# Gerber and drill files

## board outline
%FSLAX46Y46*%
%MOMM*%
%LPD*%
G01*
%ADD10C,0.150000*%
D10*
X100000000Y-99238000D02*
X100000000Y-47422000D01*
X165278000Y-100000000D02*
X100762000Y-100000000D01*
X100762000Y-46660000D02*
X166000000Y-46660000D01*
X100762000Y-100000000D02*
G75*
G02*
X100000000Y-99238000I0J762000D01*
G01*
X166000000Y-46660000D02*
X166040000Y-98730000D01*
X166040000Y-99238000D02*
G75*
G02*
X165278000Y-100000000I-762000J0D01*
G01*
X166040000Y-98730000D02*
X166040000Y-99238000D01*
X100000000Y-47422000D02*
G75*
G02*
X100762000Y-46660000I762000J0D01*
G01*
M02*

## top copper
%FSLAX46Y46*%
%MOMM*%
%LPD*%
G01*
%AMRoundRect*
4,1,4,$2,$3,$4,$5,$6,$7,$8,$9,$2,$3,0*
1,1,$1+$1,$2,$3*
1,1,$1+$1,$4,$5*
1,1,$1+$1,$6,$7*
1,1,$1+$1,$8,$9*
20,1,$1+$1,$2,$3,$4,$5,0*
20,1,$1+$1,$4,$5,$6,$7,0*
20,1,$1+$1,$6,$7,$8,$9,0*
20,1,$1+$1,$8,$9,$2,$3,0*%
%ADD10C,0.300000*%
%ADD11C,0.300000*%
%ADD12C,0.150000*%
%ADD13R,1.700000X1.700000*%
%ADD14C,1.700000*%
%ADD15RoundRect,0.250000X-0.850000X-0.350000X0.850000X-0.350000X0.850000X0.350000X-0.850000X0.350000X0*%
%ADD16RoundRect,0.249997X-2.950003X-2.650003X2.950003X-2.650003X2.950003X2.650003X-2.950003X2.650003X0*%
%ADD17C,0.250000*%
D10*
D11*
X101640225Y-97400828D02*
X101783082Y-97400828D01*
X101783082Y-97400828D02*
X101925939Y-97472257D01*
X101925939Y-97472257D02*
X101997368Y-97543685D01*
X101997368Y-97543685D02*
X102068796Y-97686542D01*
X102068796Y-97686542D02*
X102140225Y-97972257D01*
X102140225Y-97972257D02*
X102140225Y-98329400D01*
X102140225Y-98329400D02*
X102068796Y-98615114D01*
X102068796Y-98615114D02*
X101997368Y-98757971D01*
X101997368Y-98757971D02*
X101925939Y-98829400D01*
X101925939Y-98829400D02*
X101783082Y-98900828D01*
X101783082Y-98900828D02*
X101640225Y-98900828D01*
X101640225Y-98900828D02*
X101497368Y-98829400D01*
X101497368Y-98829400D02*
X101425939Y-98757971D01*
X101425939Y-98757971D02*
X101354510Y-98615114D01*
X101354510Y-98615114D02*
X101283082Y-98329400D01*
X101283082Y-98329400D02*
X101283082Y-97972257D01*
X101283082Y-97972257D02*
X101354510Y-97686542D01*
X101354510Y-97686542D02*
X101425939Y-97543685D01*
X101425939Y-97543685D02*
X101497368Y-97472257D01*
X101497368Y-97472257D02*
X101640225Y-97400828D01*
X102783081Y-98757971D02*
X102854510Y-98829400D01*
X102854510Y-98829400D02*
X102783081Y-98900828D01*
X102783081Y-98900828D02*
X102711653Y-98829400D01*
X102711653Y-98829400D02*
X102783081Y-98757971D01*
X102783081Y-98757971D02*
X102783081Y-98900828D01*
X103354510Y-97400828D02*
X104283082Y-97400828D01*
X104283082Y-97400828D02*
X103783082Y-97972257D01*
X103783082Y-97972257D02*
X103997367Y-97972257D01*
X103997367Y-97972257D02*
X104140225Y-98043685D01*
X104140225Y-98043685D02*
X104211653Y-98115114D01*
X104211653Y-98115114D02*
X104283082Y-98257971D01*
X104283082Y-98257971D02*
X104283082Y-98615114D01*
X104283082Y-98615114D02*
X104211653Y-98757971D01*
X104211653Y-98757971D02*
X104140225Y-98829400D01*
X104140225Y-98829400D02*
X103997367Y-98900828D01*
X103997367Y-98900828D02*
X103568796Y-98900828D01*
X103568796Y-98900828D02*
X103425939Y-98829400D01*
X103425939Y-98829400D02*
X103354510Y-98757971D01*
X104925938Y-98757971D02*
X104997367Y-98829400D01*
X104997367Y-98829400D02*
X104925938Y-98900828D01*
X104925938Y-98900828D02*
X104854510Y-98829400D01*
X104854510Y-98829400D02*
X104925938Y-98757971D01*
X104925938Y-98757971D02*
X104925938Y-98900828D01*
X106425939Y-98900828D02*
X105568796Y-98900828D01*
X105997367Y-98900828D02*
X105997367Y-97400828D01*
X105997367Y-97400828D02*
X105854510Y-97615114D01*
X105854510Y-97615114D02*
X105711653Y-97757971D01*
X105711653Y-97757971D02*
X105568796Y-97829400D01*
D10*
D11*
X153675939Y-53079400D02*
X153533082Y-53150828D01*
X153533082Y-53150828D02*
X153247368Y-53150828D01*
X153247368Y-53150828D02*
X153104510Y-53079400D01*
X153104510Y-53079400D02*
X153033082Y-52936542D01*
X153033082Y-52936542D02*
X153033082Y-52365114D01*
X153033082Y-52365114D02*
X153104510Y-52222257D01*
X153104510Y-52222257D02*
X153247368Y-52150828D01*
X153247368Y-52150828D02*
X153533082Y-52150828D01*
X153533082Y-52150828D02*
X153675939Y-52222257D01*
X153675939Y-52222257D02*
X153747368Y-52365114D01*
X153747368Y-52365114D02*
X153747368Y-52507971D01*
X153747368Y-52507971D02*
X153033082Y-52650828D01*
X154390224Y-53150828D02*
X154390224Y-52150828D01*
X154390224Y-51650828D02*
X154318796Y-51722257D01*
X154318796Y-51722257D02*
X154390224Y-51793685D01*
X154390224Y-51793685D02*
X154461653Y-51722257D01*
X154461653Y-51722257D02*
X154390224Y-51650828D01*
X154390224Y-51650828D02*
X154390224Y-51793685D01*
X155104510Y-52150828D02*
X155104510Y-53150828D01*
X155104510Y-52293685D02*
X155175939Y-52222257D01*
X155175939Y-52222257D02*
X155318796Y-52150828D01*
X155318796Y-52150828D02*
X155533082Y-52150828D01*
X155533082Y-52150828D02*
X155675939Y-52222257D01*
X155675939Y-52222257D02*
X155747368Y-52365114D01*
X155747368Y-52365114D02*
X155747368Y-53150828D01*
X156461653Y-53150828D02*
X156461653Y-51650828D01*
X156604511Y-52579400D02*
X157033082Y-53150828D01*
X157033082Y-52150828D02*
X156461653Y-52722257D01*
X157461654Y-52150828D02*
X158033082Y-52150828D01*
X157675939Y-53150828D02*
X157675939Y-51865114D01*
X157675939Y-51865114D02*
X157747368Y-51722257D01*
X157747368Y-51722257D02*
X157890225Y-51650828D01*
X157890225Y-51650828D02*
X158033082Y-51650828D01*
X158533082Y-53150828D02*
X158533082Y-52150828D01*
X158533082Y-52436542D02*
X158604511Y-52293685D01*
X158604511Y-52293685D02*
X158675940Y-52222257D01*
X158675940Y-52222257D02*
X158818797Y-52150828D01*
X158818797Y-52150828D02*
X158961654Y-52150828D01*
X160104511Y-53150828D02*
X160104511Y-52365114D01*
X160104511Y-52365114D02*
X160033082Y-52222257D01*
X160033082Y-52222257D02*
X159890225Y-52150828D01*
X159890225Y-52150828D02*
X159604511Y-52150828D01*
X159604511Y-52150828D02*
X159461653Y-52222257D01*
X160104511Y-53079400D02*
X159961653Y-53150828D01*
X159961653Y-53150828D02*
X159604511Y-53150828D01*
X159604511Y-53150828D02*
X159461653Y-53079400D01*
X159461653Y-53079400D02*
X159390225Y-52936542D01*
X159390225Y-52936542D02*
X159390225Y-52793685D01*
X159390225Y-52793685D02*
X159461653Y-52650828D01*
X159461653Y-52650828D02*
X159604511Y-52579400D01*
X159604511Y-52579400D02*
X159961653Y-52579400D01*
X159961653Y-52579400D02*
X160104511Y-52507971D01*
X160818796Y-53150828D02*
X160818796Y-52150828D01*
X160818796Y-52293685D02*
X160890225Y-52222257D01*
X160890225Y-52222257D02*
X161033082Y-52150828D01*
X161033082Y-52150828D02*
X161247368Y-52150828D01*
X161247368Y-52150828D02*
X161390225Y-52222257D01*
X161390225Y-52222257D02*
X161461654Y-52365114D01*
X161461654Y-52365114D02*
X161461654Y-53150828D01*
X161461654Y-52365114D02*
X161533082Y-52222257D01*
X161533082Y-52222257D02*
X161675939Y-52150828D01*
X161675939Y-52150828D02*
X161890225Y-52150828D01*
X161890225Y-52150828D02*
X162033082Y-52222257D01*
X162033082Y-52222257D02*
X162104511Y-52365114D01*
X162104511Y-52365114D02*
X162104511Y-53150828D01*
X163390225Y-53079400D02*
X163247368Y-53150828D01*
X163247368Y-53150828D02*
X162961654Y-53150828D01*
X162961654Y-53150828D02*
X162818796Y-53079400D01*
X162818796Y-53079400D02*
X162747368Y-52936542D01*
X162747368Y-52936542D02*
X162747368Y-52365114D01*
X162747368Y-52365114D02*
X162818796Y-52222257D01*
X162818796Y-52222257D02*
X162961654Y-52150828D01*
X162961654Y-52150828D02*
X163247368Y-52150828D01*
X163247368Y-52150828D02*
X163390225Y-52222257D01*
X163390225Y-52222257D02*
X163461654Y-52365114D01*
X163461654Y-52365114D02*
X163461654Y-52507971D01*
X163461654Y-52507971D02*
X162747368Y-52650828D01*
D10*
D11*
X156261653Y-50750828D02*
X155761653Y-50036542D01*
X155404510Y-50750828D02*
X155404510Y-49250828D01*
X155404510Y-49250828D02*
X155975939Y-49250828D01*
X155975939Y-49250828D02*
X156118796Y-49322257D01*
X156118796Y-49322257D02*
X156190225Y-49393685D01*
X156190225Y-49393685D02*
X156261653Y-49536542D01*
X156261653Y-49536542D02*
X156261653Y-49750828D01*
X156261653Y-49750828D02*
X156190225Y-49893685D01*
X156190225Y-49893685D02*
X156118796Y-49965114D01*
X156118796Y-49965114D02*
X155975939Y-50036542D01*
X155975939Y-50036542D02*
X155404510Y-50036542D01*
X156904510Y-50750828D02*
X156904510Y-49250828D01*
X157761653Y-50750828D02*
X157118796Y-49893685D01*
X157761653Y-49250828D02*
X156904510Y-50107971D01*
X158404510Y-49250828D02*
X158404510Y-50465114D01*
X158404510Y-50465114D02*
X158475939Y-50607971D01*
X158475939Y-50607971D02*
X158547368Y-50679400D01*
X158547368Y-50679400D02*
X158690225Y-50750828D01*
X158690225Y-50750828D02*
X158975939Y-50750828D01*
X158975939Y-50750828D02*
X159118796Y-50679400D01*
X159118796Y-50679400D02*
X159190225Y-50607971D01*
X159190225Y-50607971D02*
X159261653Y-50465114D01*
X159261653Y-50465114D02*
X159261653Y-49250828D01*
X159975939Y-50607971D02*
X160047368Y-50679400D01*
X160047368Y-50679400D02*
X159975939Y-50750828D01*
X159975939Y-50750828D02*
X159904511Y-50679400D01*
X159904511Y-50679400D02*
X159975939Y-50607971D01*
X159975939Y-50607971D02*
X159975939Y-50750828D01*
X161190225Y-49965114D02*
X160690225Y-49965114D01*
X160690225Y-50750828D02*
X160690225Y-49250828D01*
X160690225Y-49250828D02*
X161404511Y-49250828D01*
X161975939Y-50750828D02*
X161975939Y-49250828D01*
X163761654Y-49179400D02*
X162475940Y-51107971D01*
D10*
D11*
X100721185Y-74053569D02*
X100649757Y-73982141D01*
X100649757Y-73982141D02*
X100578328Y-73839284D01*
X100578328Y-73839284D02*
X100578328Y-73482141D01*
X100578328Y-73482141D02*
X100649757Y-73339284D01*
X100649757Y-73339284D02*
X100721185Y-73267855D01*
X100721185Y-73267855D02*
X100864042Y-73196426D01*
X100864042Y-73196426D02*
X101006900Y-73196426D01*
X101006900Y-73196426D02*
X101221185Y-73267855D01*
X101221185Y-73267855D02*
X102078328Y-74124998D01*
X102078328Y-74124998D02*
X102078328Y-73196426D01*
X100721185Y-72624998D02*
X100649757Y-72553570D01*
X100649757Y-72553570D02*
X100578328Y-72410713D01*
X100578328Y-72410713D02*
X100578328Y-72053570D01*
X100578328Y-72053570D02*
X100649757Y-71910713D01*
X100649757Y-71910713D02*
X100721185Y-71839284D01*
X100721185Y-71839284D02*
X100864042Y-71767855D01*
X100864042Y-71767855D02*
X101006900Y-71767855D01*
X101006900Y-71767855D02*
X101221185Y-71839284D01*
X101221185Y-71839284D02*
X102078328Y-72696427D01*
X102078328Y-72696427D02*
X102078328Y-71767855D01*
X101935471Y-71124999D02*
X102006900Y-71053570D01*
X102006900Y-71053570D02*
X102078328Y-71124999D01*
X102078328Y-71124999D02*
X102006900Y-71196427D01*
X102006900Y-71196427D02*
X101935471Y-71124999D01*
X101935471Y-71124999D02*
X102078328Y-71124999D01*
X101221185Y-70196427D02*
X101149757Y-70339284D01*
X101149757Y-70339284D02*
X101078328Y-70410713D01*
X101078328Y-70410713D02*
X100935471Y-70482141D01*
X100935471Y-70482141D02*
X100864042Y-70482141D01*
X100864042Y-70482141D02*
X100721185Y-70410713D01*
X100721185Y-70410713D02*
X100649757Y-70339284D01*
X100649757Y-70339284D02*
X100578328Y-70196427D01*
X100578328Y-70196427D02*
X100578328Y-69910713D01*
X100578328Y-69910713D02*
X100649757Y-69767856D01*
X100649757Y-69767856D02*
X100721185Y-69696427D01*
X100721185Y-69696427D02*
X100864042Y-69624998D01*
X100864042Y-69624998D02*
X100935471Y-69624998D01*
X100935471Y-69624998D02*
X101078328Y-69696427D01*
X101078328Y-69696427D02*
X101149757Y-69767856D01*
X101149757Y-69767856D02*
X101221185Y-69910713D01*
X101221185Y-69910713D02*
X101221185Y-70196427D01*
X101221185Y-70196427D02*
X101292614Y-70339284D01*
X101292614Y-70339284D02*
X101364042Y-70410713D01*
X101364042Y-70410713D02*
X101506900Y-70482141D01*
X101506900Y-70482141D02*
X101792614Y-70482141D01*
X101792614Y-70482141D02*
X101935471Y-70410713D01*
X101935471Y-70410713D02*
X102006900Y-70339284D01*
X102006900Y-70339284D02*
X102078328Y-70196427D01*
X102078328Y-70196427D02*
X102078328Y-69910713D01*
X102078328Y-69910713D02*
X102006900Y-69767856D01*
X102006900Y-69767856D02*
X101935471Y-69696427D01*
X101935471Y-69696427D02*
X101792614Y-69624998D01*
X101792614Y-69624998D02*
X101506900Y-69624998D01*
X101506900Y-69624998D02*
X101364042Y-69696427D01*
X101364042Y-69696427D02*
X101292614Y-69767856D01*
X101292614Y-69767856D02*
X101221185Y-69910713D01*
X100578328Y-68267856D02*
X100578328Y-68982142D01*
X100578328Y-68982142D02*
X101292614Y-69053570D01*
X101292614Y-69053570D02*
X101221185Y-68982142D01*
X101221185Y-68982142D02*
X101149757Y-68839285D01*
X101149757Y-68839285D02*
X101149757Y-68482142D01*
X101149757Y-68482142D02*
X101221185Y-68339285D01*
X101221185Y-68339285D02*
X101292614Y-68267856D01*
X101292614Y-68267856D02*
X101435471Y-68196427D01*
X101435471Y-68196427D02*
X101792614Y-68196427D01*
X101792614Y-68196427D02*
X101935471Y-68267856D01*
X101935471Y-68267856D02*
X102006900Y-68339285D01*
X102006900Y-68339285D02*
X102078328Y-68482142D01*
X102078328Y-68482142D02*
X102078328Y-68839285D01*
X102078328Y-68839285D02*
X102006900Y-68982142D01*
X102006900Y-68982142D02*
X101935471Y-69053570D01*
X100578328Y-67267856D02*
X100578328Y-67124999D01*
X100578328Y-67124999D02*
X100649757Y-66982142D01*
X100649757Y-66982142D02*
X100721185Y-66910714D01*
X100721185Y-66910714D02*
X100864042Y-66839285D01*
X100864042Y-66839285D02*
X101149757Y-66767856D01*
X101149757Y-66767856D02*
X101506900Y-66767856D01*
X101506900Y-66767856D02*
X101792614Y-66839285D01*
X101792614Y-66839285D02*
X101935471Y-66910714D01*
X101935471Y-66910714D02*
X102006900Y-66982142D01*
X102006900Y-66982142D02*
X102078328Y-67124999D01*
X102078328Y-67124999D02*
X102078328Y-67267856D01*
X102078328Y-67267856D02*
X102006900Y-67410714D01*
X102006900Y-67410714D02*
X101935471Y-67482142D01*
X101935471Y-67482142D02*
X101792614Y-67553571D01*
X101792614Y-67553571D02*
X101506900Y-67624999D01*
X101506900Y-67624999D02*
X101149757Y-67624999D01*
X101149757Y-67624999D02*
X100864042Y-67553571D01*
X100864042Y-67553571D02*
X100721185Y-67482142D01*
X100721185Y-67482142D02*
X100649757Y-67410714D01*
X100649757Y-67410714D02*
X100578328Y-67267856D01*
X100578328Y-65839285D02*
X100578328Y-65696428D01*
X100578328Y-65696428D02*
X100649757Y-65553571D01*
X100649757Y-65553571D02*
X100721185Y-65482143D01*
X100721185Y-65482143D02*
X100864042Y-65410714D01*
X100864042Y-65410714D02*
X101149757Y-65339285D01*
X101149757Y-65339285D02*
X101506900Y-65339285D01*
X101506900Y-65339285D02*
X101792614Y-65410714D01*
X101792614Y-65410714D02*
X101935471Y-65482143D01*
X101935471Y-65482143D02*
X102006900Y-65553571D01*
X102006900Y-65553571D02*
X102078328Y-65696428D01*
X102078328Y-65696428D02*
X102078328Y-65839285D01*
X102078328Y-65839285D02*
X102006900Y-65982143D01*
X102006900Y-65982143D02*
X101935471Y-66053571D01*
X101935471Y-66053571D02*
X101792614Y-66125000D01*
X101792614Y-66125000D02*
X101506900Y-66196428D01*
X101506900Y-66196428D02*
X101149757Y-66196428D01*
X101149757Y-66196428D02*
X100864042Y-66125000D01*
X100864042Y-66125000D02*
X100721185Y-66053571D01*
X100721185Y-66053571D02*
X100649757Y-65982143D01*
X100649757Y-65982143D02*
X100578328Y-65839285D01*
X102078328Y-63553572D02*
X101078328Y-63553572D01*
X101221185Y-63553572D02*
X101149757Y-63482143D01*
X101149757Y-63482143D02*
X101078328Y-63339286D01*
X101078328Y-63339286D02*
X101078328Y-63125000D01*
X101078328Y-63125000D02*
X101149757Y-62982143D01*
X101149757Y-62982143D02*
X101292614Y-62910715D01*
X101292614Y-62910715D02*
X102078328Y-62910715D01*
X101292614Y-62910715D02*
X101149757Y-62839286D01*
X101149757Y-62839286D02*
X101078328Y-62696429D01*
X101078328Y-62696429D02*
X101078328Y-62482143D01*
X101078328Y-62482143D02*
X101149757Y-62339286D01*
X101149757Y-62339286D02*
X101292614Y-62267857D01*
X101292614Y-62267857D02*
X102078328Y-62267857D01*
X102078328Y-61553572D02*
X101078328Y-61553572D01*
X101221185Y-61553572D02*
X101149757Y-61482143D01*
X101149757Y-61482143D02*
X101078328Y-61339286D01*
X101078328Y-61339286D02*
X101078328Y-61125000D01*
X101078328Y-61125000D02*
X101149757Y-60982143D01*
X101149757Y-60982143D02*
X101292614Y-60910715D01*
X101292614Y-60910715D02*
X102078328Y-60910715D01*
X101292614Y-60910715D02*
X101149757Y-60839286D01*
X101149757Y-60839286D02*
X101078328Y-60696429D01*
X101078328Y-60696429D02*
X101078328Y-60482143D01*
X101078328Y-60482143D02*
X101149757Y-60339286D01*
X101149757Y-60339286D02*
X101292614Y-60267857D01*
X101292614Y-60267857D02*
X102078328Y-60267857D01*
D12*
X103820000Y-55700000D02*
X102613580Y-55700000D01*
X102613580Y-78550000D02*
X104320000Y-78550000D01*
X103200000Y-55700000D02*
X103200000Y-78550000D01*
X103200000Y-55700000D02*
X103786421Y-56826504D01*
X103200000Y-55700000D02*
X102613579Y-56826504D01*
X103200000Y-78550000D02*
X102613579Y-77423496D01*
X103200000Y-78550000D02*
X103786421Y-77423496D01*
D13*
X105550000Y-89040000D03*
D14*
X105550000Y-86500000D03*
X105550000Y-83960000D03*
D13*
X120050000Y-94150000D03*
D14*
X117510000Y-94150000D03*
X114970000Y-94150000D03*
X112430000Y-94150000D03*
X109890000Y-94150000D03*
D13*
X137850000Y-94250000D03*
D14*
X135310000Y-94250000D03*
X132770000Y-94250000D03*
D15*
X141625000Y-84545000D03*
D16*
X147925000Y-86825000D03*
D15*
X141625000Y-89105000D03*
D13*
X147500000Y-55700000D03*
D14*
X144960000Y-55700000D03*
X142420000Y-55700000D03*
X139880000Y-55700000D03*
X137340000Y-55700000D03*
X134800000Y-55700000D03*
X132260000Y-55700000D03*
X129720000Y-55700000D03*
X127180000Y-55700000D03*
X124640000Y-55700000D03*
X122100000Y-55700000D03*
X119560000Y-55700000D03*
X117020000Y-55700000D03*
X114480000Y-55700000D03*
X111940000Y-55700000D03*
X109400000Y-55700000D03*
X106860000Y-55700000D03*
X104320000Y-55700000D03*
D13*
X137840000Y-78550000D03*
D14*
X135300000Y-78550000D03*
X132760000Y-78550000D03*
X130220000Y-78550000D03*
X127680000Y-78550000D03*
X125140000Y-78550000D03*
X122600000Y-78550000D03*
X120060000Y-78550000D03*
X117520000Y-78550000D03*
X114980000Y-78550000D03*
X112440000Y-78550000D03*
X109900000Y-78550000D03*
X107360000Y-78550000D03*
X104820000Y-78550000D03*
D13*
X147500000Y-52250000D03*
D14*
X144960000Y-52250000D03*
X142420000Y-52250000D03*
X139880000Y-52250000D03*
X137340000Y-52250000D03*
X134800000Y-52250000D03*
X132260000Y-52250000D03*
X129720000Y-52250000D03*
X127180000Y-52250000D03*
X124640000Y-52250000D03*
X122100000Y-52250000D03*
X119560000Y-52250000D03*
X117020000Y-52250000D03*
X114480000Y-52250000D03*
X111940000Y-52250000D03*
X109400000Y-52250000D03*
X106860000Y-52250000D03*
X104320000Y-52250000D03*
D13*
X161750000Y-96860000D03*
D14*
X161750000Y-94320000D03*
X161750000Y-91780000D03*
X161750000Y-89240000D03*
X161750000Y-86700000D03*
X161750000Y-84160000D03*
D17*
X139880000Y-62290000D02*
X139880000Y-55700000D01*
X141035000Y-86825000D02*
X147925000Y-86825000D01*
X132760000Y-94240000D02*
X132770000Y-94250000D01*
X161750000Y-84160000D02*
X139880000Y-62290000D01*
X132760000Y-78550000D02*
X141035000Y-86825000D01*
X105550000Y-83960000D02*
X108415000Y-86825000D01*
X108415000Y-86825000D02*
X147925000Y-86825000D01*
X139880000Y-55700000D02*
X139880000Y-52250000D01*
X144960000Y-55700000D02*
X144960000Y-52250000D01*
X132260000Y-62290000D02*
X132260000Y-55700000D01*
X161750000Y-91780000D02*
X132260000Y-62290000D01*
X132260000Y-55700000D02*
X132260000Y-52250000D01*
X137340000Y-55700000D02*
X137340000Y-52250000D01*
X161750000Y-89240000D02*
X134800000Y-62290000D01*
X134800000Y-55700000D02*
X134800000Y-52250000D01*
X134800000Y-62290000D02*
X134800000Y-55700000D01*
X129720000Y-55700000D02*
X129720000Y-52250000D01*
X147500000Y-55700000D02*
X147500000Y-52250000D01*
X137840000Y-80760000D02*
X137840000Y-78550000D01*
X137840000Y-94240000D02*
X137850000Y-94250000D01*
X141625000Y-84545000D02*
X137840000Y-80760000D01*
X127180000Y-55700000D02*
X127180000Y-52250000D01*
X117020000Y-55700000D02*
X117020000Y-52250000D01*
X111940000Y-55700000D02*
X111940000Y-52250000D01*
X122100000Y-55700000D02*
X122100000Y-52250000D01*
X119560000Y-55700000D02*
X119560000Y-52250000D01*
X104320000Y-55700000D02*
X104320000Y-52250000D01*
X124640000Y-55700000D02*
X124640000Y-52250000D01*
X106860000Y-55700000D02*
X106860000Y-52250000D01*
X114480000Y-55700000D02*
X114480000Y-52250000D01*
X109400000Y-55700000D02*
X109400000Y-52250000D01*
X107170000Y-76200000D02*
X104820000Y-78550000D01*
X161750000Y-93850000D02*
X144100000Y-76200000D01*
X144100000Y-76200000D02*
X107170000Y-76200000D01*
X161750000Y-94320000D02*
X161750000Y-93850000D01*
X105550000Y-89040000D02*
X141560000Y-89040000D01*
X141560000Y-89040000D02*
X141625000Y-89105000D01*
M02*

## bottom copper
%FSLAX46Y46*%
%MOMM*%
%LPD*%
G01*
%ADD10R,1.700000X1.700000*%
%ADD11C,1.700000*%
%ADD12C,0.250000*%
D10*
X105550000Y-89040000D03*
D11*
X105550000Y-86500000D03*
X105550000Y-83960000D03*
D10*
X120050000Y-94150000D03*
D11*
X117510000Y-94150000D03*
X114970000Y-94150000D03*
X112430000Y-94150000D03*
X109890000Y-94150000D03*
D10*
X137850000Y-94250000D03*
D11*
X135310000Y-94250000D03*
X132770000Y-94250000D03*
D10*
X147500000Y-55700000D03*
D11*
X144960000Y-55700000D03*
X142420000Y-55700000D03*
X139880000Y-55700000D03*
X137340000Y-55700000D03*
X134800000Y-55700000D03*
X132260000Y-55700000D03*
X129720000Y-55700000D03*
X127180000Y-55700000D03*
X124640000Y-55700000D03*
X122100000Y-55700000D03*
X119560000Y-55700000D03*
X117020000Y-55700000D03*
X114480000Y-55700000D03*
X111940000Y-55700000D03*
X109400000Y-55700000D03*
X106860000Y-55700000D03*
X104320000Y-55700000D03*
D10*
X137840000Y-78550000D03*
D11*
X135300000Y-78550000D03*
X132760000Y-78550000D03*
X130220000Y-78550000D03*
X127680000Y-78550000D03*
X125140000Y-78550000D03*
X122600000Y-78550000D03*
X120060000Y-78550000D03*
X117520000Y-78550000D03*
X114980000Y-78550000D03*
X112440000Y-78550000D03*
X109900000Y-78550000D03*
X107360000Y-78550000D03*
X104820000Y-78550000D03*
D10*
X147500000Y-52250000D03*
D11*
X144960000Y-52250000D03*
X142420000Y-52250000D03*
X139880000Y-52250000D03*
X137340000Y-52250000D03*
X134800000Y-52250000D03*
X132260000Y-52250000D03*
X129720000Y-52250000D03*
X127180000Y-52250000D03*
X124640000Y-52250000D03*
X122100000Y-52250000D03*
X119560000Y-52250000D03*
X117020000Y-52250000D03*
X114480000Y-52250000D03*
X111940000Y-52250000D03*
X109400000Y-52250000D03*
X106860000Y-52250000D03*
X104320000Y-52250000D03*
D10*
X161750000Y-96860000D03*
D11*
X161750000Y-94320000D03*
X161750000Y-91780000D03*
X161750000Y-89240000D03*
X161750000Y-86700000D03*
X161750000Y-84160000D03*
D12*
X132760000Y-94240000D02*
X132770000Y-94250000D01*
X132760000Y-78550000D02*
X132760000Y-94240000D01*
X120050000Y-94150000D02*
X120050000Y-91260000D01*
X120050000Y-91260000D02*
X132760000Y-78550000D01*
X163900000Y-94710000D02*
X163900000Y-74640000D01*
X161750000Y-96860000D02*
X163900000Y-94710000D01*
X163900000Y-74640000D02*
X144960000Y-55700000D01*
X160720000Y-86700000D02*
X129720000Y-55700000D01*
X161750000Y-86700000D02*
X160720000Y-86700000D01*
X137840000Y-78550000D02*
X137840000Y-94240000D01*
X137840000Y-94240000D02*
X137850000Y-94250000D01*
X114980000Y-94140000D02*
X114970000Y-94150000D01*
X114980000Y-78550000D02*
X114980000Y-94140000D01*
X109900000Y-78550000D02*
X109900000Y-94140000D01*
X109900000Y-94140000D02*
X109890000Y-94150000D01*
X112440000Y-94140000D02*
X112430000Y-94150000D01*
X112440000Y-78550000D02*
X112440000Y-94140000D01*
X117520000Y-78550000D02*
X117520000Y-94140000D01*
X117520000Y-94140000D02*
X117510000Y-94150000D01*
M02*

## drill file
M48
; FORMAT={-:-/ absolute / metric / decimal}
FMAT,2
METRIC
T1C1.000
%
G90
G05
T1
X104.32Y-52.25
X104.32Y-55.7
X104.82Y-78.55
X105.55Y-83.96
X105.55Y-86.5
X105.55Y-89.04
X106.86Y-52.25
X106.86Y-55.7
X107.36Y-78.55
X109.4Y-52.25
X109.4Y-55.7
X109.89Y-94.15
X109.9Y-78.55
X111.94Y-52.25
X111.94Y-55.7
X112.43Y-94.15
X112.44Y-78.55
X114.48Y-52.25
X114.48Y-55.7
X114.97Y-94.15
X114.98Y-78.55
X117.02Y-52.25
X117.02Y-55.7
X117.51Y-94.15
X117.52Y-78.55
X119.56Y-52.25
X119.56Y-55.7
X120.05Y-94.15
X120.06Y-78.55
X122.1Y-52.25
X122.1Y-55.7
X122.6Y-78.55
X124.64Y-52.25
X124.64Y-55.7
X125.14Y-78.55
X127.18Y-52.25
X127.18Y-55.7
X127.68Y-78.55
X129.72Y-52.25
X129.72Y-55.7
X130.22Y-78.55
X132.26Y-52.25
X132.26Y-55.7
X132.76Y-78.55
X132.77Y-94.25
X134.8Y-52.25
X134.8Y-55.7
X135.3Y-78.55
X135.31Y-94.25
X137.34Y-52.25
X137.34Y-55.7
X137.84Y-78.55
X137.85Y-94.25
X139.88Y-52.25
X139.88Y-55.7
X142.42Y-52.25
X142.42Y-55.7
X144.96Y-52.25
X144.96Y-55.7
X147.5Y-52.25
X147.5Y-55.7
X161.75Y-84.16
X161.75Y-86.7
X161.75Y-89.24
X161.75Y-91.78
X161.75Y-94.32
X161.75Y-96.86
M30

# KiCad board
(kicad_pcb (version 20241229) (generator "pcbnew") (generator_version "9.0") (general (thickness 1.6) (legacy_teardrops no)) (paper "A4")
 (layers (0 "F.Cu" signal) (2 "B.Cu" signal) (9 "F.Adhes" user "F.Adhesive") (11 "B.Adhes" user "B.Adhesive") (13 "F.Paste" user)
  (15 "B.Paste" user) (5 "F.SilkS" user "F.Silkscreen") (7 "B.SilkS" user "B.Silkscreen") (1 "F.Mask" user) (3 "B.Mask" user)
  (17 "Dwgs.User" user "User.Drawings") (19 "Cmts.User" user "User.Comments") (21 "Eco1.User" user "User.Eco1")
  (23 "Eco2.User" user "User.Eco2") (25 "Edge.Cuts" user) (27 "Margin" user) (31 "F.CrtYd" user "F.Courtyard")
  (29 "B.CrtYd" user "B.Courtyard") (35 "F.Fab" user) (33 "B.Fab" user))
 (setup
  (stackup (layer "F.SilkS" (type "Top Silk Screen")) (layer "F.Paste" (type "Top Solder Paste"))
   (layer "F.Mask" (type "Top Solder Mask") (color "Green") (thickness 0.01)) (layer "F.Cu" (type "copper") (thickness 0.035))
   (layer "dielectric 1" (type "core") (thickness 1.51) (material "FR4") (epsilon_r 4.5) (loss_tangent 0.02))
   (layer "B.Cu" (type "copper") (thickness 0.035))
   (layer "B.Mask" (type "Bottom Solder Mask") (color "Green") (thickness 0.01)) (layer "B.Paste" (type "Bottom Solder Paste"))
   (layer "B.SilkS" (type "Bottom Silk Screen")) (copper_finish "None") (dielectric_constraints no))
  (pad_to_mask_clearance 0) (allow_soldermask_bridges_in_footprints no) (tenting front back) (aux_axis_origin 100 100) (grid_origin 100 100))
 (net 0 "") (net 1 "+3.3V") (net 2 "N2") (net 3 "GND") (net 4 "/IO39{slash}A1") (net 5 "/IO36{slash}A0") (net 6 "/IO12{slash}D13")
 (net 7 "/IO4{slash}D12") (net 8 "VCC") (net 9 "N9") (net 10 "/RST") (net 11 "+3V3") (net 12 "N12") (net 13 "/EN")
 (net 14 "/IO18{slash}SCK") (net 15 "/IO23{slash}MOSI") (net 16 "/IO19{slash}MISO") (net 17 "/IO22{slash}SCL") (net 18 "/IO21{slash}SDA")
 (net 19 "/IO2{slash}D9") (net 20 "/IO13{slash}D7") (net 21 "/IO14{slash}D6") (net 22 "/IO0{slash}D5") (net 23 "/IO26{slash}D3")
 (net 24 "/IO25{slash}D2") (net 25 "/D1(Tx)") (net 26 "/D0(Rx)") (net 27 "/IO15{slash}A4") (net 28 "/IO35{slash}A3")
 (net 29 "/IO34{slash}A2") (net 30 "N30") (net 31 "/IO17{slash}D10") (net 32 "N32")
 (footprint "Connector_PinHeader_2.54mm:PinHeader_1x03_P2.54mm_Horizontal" (layer "F.Cu") (at 105.55 89.04 180)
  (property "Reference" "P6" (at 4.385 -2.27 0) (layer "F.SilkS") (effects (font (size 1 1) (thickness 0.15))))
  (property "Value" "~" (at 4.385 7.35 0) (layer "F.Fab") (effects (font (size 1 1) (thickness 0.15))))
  (pad "1" thru_hole rect (at 0 0 180) (size 1.7 1.7) (drill 1) (layers "*.Cu" "*.Mask") (remove_unused_layers no) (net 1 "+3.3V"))
  (pad "2" thru_hole circle (at 0 2.54 180) (size 1.7 1.7) (drill 1) (layers "*.Cu" "*.Mask") (remove_unused_layers no) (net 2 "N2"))
  (pad "3" thru_hole circle (at 0 5.08 180) (size 1.7 1.7) (drill 1) (layers "*.Cu" "*.Mask") (remove_unused_layers no) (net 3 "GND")))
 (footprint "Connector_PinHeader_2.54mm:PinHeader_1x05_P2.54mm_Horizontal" (layer "F.Cu") (at 120.05 94.15 -90)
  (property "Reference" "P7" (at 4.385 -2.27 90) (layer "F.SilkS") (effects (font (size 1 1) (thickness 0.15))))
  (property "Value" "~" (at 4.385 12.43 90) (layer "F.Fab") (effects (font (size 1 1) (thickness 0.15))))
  (pad "1" thru_hole rect (at 0 0 270) (size 1.7 1.7) (drill 1) (layers "*.Cu" "*.Mask") (remove_unused_layers no) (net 3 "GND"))
  (pad "2" thru_hole circle (at 0 2.54 270) (size 1.7 1.7) (drill 1) (layers "*.Cu" "*.Mask") (remove_unused_layers no)
   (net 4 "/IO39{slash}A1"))
  (pad "3" thru_hole circle (at 0 5.08 270) (size 1.7 1.7) (drill 1) (layers "*.Cu" "*.Mask") (remove_unused_layers no)
   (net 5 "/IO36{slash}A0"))
  (pad "4" thru_hole circle (at 0 7.62 270) (size 1.7 1.7) (drill 1) (layers "*.Cu" "*.Mask") (remove_unused_layers no)
   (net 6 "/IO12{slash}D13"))
  (pad "5" thru_hole circle (at 0 10.16 270) (size 1.7 1.7) (drill 1) (layers "*.Cu" "*.Mask") (remove_unused_layers no)
   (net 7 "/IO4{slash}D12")))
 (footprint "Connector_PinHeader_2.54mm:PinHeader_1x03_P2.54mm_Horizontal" (layer "F.Cu") (at 137.85 94.25 -90)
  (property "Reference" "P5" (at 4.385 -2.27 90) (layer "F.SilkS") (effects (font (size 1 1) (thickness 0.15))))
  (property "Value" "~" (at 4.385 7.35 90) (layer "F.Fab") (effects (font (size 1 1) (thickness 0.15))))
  (pad "1" thru_hole rect (at 0 0 270) (size 1.7 1.7) (drill 1) (layers "*.Cu" "*.Mask") (remove_unused_layers no) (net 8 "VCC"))
  (pad "2" thru_hole circle (at 0 2.54 270) (size 1.7 1.7) (drill 1) (layers "*.Cu" "*.Mask") (remove_unused_layers no) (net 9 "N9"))
  (pad "3" thru_hole circle (at 0 5.08 270) (size 1.7 1.7) (drill 1) (layers "*.Cu" "*.Mask") (remove_unused_layers no) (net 3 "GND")))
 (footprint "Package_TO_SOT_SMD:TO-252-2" (layer "F.Cu") (at 146.665 86.825)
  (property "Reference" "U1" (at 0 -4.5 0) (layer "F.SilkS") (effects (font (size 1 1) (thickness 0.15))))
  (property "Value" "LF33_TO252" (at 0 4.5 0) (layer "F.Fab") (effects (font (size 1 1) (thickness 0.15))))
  (pad "" smd roundrect (at -0.415 -1.525) (size 3.05 2.75) (layers "F.Paste") (roundrect_rratio 0.090909))
  (pad "" smd roundrect (at -0.415 1.525) (size 3.05 2.75) (layers "F.Paste") (roundrect_rratio 0.090909))
  (pad "" smd roundrect (at 2.935 -1.525) (size 3.05 2.75) (layers "F.Paste") (roundrect_rratio 0.090909))
  (pad "" smd roundrect (at 2.935 1.525) (size 3.05 2.75) (layers "F.Paste") (roundrect_rratio 0.090909))
  (pad "1" smd roundrect (at -5.04 -2.28) (size 2.2 1.2) (layers "F.Cu" "F.Mask" "F.Paste") (roundrect_rratio 0.208333) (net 8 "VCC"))
  (pad "2" smd roundrect (at 1.26 0) (size 6.4 5.8) (layers "F.Cu" "F.Mask") (roundrect_rratio 0.043103) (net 3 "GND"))
  (pad "3" smd roundrect (at -5.04 2.28) (size 2.2 1.2) (layers "F.Cu" "F.Mask" "F.Paste") (roundrect_rratio 0.208333) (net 1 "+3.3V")))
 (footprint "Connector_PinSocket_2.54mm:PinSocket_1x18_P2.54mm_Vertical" (layer "F.Cu") (at 147.5 55.7 -90)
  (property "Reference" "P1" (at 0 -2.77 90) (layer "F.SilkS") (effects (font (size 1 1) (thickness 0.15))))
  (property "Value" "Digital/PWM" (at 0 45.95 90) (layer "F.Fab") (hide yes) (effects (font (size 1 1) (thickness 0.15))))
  (pad "1" thru_hole rect (at 0 0 270) (size 1.7 1.7) (drill 1) (layers "*.Cu" "*.Mask") (remove_unused_layers no) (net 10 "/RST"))
  (pad "2" thru_hole circle (at 0 2.54 270) (size 1.7 1.7) (drill 1) (layers "*.Cu" "*.Mask") (remove_unused_layers no) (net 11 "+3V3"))
  (pad "3" thru_hole circle (at 0 5.08 270) (size 1.7 1.7) (drill 1) (layers "*.Cu" "*.Mask") (remove_unused_layers no) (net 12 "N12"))
  (pad "4" thru_hole circle (at 0 7.62 270) (size 1.7 1.7) (drill 1) (layers "*.Cu" "*.Mask") (remove_unused_layers no) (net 3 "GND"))
  (pad "5" thru_hole circle (at 0 10.16 270) (size 1.7 1.7) (drill 1) (layers "*.Cu" "*.Mask") (remove_unused_layers no) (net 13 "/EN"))
  (pad "6" thru_hole circle (at 0 12.7 270) (size 1.7 1.7) (drill 1) (layers "*.Cu" "*.Mask") (remove_unused_layers no)
   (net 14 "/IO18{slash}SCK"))
  (pad "7" thru_hole circle (at 0 15.24 270) (size 1.7 1.7) (drill 1) (layers "*.Cu" "*.Mask") (remove_unused_layers no)
   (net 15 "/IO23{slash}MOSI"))
  (pad "8" thru_hole circle (at 0 17.78 270) (size 1.7 1.7) (drill 1) (layers "*.Cu" "*.Mask") (remove_unused_layers no)
   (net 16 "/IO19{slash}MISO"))
  (pad "9" thru_hole circle (at 0 20.32 270) (size 1.7 1.7) (drill 1) (layers "*.Cu" "*.Mask") (remove_unused_layers no)
   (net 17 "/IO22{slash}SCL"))
  (pad "10" thru_hole circle (at 0 22.86 270) (size 1.7 1.7) (drill 1) (layers "*.Cu" "*.Mask") (remove_unused_layers no)
   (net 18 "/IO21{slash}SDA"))
  (pad "11" thru_hole circle (at 0 25.4 270) (size 1.7 1.7) (drill 1) (layers "*.Cu" "*.Mask") (remove_unused_layers no)
   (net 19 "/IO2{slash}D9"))
  (pad "12" thru_hole circle (at 0 27.94 270) (size 1.7 1.7) (drill 1) (layers "*.Cu" "*.Mask") (remove_unused_layers no)
   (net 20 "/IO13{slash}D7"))
  (pad "13" thru_hole circle (at 0 30.48 270) (size 1.7 1.7) (drill 1) (layers "*.Cu" "*.Mask") (remove_unused_layers no)
   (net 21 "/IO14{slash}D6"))
  (pad "14" thru_hole circle (at 0 33.02 270) (size 1.7 1.7) (drill 1) (layers "*.Cu" "*.Mask") (remove_unused_layers no)
   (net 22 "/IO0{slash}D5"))
  (pad "15" thru_hole circle (at 0 35.56 270) (size 1.7 1.7) (drill 1) (layers "*.Cu" "*.Mask") (remove_unused_layers no)
   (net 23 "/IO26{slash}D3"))
  (pad "16" thru_hole circle (at 0 38.1 270) (size 1.7 1.7) (drill 1) (layers "*.Cu" "*.Mask") (remove_unused_layers no)
   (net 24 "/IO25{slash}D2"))
  (pad "17" thru_hole circle (at 0 40.64 270) (size 1.7 1.7) (drill 1) (layers "*.Cu" "*.Mask") (remove_unused_layers no) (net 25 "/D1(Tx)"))
  (pad "18" thru_hole circle (at 0 43.18 270) (size 1.7 1.7) (drill 1) (layers "*.Cu" "*.Mask") (remove_unused_layers no) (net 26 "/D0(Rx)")))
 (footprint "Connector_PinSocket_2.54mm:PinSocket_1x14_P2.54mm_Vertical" (layer "F.Cu") (at 137.84 78.55 -90)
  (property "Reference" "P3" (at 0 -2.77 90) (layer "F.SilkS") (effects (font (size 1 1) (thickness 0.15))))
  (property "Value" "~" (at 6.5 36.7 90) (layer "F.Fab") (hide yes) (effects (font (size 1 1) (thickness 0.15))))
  (pad "1" thru_hole rect (at 0 0 270) (size 1.7 1.7) (drill 1) (layers "*.Cu" "*.Mask") (remove_unused_layers no) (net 8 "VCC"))
  (pad "2" thru_hole circle (at 0 2.54 270) (size 1.7 1.7) (drill 1) (layers "*.Cu" "*.Mask") (remove_unused_layers no) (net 11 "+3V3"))
  (pad "3" thru_hole circle (at 0 5.08 270) (size 1.7 1.7) (drill 1) (layers "*.Cu" "*.Mask") (remove_unused_layers no) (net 3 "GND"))
  (pad "4" thru_hole circle (at 0 7.62 270) (size 1.7 1.7) (drill 1) (layers "*.Cu" "*.Mask") (remove_unused_layers no)
   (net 17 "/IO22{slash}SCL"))
  (pad "5" thru_hole circle (at 0 10.16 270) (size 1.7 1.7) (drill 1) (layers "*.Cu" "*.Mask") (remove_unused_layers no)
   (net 18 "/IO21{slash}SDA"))
  (pad "6" thru_hole circle (at 0 12.7 270) (size 1.7 1.7) (drill 1) (layers "*.Cu" "*.Mask") (remove_unused_layers no)
   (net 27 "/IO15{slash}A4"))
  (pad "7" thru_hole circle (at 0 15.24 270) (size 1.7 1.7) (drill 1) (layers "*.Cu" "*.Mask") (remove_unused_layers no)
   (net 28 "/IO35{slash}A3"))
  (pad "8" thru_hole circle (at 0 17.78 270) (size 1.7 1.7) (drill 1) (layers "*.Cu" "*.Mask") (remove_unused_layers no)
   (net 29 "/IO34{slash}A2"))
  (pad "9" thru_hole circle (at 0 20.32 270) (size 1.7 1.7) (drill 1) (layers "*.Cu" "*.Mask") (remove_unused_layers no)
   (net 4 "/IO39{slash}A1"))
  (pad "10" thru_hole circle (at 0 22.86 270) (size 1.7 1.7) (drill 1) (layers "*.Cu" "*.Mask") (remove_unused_layers no)
   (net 5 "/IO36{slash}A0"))
  (pad "11" thru_hole circle (at 0 25.4 270) (size 1.7 1.7) (drill 1) (layers "*.Cu" "*.Mask") (remove_unused_layers no)
   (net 6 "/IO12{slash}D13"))
  (pad "12" thru_hole circle (at 0 27.94 270) (size 1.7 1.7) (drill 1) (layers "*.Cu" "*.Mask") (remove_unused_layers no)
   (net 7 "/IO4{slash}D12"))
  (pad "13" thru_hole circle (at 0 30.48 270) (size 1.7 1.7) (drill 1) (layers "*.Cu" "*.Mask") (remove_unused_layers no) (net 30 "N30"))
  (pad "14" thru_hole circle (at 0 33.02 270) (size 1.7 1.7) (drill 1) (layers "*.Cu" "*.Mask") (remove_unused_layers no)
   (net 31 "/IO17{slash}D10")))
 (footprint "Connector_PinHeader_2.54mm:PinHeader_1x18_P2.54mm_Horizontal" (layer "B.Cu") (at 147.5 52.25 90)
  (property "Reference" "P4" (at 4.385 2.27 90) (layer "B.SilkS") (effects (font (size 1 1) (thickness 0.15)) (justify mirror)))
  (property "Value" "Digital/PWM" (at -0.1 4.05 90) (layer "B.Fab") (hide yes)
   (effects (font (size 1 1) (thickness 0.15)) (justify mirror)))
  (pad "1" thru_hole rect (at 0 0 90) (size 1.7 1.7) (drill 1) (layers "*.Cu" "*.Mask") (remove_unused_layers no) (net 10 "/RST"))
  (pad "2" thru_hole circle (at 0 -2.54 90) (size 1.7 1.7) (drill 1) (layers "*.Cu" "*.Mask") (remove_unused_layers no) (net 11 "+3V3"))
  (pad "3" thru_hole circle (at 0 -5.08 90) (size 1.7 1.7) (drill 1) (layers "*.Cu" "*.Mask") (remove_unused_layers no) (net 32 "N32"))
  (pad "4" thru_hole circle (at 0 -7.62 90) (size 1.7 1.7) (drill 1) (layers "*.Cu" "*.Mask") (remove_unused_layers no) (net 3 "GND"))
  (pad "5" thru_hole circle (at 0 -10.16 90) (size 1.7 1.7) (drill 1) (layers "*.Cu" "*.Mask") (remove_unused_layers no) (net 13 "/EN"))
  (pad "6" thru_hole circle (at 0 -12.7 90) (size 1.7 1.7) (drill 1) (layers "*.Cu" "*.Mask") (remove_unused_layers no)
   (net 14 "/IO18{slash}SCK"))
  (pad "7" thru_hole circle (at 0 -15.24 90) (size 1.7 1.7) (drill 1) (layers "*.Cu" "*.Mask") (remove_unused_layers no)
   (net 15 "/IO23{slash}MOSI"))
  (pad "8" thru_hole circle (at 0 -17.78 90) (size 1.7 1.7) (drill 1) (layers "*.Cu" "*.Mask") (remove_unused_layers no)
   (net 16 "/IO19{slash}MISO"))
  (pad "9" thru_hole circle (at 0 -20.32 90) (size 1.7 1.7) (drill 1) (layers "*.Cu" "*.Mask") (remove_unused_layers no)
   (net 17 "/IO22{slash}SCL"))
  (pad "10" thru_hole circle (at 0 -22.86 90) (size 1.7 1.7) (drill 1) (layers "*.Cu" "*.Mask") (remove_unused_layers no)
   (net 18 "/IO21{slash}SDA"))
  (pad "11" thru_hole circle (at 0 -25.4 90) (size 1.7 1.7) (drill 1) (layers "*.Cu" "*.Mask") (remove_unused_layers no)
   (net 19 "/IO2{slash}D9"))
  (pad "12" thru_hole circle (at 0 -27.94 90) (size 1.7 1.7) (drill 1) (layers "*.Cu" "*.Mask") (remove_unused_layers no)
   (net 20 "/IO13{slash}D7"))
  (pad "13" thru_hole circle (at 0 -30.48 90) (size 1.7 1.7) (drill 1) (layers "*.Cu" "*.Mask") (remove_unused_layers no)
   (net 21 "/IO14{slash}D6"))
  (pad "14" thru_hole circle (at 0 -33.02 90) (size 1.7 1.7) (drill 1) (layers "*.Cu" "*.Mask") (remove_unused_layers no)
   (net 22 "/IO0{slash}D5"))
  (pad "15" thru_hole circle (at 0 -35.56 90) (size 1.7 1.7) (drill 1) (layers "*.Cu" "*.Mask") (remove_unused_layers no)
   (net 23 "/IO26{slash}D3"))
  (pad "16" thru_hole circle (at 0 -38.1 90) (size 1.7 1.7) (drill 1) (layers "*.Cu" "*.Mask") (remove_unused_layers no)
   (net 24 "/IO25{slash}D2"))
  (pad "17" thru_hole circle (at 0 -40.64 90) (size 1.7 1.7) (drill 1) (layers "*.Cu" "*.Mask") (remove_unused_layers no) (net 25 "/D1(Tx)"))
  (pad "18" thru_hole circle (at 0 -43.18 90) (size 1.7 1.7) (drill 1) (layers "*.Cu" "*.Mask") (remove_unused_layers no) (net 26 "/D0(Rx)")))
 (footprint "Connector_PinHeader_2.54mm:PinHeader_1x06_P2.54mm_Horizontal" (layer "B.Cu") (at 161.75 96.86)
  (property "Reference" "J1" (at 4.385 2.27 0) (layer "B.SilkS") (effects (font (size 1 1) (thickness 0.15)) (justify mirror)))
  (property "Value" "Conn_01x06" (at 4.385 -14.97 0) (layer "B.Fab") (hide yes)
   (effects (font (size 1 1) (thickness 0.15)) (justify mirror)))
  (pad "1" thru_hole rect (at 0 0) (size 1.7 1.7) (drill 1) (layers "*.Cu" "*.Mask") (remove_unused_layers no) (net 11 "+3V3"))
  (pad "2" thru_hole circle (at 0 -2.54) (size 1.7 1.7) (drill 1) (layers "*.Cu" "*.Mask") (remove_unused_layers no)
   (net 31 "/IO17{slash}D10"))
  (pad "3" thru_hole circle (at 0 -5.08) (size 1.7 1.7) (drill 1) (layers "*.Cu" "*.Mask") (remove_unused_layers no)
   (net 15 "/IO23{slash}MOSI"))
  (pad "4" thru_hole circle (at 0 -7.62) (size 1.7 1.7) (drill 1) (layers "*.Cu" "*.Mask") (remove_unused_layers no)
   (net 14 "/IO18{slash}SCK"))
  (pad "5" thru_hole circle (at 0 -10.16) (size 1.7 1.7) (drill 1) (layers "*.Cu" "*.Mask") (remove_unused_layers no)
   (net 16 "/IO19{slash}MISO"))
  (pad "6" thru_hole circle (at 0 -12.7) (size 1.7 1.7) (drill 1) (layers "*.Cu" "*.Mask") (remove_unused_layers no) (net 3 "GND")))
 (gr_line (start 100 99.238) (end 100 47.422) (stroke (width 0.15) (type solid)) (layer "Edge.Cuts"))
 (gr_line (start 165.278 100) (end 100.762 100) (stroke (width 0.15) (type solid)) (layer "Edge.Cuts"))
 (gr_line (start 100.762 46.66) (end 166 46.66) (stroke (width 0.15) (type solid)) (layer "Edge.Cuts"))
 (gr_arc (start 100.762 100) (mid 100.223185 99.776815) (end 100 99.238) (stroke (width 0.15) (type solid)) (layer "Edge.Cuts"))
 (gr_line (start 166 46.66) (end 166.04 98.73) (stroke (width 0.15) (type solid)) (layer "Edge.Cuts"))
 (gr_arc (start 166.04 99.238) (mid 165.816815 99.776815) (end 165.278 100) (stroke (width 0.15) (type solid)) (layer "Edge.Cuts"))
 (gr_line (start 166.04 98.73) (end 166.04 99.238) (stroke (width 0.15) (type solid)) (layer "Edge.Cuts"))
 (gr_arc (start 100 47.422) (mid 100.223185 46.883185) (end 100.762 46.66) (stroke (width 0.15) (type solid)) (layer "Edge.Cuts"))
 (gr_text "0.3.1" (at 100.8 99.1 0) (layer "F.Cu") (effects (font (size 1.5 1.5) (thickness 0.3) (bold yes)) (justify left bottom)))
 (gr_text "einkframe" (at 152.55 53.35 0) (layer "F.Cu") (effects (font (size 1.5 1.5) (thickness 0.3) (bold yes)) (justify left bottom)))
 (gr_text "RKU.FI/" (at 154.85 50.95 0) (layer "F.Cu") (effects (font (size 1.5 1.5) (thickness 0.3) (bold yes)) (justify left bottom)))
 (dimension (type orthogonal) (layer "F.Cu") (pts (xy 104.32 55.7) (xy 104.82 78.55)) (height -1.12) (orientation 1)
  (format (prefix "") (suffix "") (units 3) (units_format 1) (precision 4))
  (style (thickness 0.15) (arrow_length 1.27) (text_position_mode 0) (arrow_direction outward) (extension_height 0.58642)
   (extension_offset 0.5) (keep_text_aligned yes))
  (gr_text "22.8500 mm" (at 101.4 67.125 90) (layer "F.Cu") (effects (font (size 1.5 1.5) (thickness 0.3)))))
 (segment (start 139.88 62.29) (end 139.88 55.7) (width 0.25) (layer "F.Cu") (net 3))
 (segment (start 141.035 86.825) (end 147.925 86.825) (width 0.25) (layer "F.Cu") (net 3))
 (segment (start 132.76 94.24) (end 132.77 94.25) (width 0.25) (layer "F.Cu") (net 3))
 (segment (start 161.75 84.16) (end 139.88 62.29) (width 0.25) (layer "F.Cu") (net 3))
 (segment (start 132.76 78.55) (end 141.035 86.825) (width 0.25) (layer "F.Cu") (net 3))
 (segment (start 105.55 83.96) (end 108.415 86.825) (width 0.25) (layer "F.Cu") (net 3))
 (segment (start 108.415 86.825) (end 147.925 86.825) (width 0.25) (layer "F.Cu") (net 3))
 (segment (start 139.88 55.7) (end 139.88 52.25) (width 0.25) (layer "F.Cu") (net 3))
 (segment (start 132.76 94.24) (end 132.77 94.25) (width 0.25) (layer "B.Cu") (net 3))
 (segment (start 132.76 78.55) (end 132.76 94.24) (width 0.25) (layer "B.Cu") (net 3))
 (segment (start 120.05 94.15) (end 120.05 91.26) (width 0.25) (layer "B.Cu") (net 3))
 (segment (start 120.05 91.26) (end 132.76 78.55) (width 0.25) (layer "B.Cu") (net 3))
 (segment (start 144.96 55.7) (end 144.96 52.25) (width 0.25) (layer "F.Cu") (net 11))
 (segment (start 163.9 94.71) (end 163.9 74.64) (width 0.25) (layer "B.Cu") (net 11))
 (segment (start 161.75 96.86) (end 163.9 94.71) (width 0.25) (layer "B.Cu") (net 11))
 (segment (start 163.9 74.64) (end 144.96 55.7) (width 0.25) (layer "B.Cu") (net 11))
 (segment (start 132.26 62.29) (end 132.26 55.7) (width 0.25) (layer "F.Cu") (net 15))
 (segment (start 161.75 91.78) (end 132.26 62.29) (width 0.25) (layer "F.Cu") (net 15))
 (segment (start 132.26 55.7) (end 132.26 52.25) (width 0.25) (layer "F.Cu") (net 15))
 (segment (start 137.34 55.7) (end 137.34 52.25) (width 0.25) (layer "F.Cu") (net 13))
 (segment (start 161.75 89.24) (end 134.8 62.29) (width 0.25) (layer "F.Cu") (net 14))
 (segment (start 134.8 55.7) (end 134.8 52.25) (width 0.25) (layer "F.Cu") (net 14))
 (segment (start 134.8 62.29) (end 134.8 55.7) (width 0.25) (layer "F.Cu") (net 14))
 (segment (start 129.72 55.7) (end 129.72 52.25) (width 0.25) (layer "F.Cu") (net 16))
 (segment (start 160.72 86.7) (end 129.72 55.7) (width 0.25) (layer "B.Cu") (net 16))
 (segment (start 161.75 86.7) (end 160.72 86.7) (width 0.25) (layer "B.Cu") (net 16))
 (segment (start 147.5 55.7) (end 147.5 52.25) (width 0.25) (layer "F.Cu") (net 10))
 (segment (start 137.84 80.76) (end 137.84 78.55) (width 0.25) (layer "F.Cu") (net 8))
 (segment (start 137.84 94.24) (end 137.85 94.25) (width 0.25) (layer "F.Cu") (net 8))
 (segment (start 141.625 84.545) (end 137.84 80.76) (width 0.25) (layer "F.Cu") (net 8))
 (segment (start 137.84 78.55) (end 137.84 94.24) (width 0.25) (layer "B.Cu") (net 8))
 (segment (start 137.84 94.24) (end 137.85 94.25) (width 0.25) (layer "B.Cu") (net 8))
 (segment (start 127.18 55.7) (end 127.18 52.25) (width 0.25) (layer "F.Cu") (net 17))
 (segment (start 117.02 55.7) (end 117.02 52.25) (width 0.25) (layer "F.Cu") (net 21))
 (segment (start 111.94 55.7) (end 111.94 52.25) (width 0.25) (layer "F.Cu") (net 23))
 (segment (start 122.1 55.7) (end 122.1 52.25) (width 0.25) (layer "F.Cu") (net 19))
 (segment (start 119.56 55.7) (end 119.56 52.25) (width 0.25) (layer "F.Cu") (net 20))
 (segment (start 104.32 55.7) (end 104.32 52.25) (width 0.25) (layer "F.Cu") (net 26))
 (segment (start 124.64 55.7) (end 124.64 52.25) (width 0.25) (layer "F.Cu") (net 18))
 (segment (start 106.86 55.7) (end 106.86 52.25) (width 0.25) (layer "F.Cu") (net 25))
 (segment (start 114.48 55.7) (end 114.48 52.25) (width 0.25) (layer "F.Cu") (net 22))
 (segment (start 109.4 55.7) (end 109.4 52.25) (width 0.25) (layer "F.Cu") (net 24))
 (segment (start 114.98 94.14) (end 114.97 94.15) (width 0.25) (layer "B.Cu") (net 5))
 (segment (start 114.98 78.55) (end 114.98 94.14) (width 0.25) (layer "B.Cu") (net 5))
 (segment (start 109.9 78.55) (end 109.9 94.14) (width 0.25) (layer "B.Cu") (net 7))
 (segment (start 109.9 94.14) (end 109.89 94.15) (width 0.25) (layer "B.Cu") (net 7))
 (segment (start 107.17 76.2) (end 104.82 78.55) (width 0.25) (layer "F.Cu") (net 31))
 (segment (start 161.75 93.85) (end 144.1 76.2) (width 0.25) (layer "F.Cu") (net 31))
 (segment (start 144.1 76.2) (end 107.17 76.2) (width 0.25) (layer "F.Cu") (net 31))
 (segment (start 161.75 94.32) (end 161.75 93.85) (width 0.25) (layer "F.Cu") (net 31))
 (segment (start 112.44 94.14) (end 112.43 94.15) (width 0.25) (layer "B.Cu") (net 6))
 (segment (start 112.44 78.55) (end 112.44 94.14) (width 0.25) (layer "B.Cu") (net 6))
 (segment (start 117.52 78.55) (end 117.52 94.14) (width 0.25) (layer "B.Cu") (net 4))
 (segment (start 117.52 94.14) (end 117.51 94.15) (width 0.25) (layer "B.Cu") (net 4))
 (segment (start 105.55 89.04) (end 141.56 89.04) (width 0.25) (layer "F.Cu") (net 1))
 (segment (start 141.56 89.04) (end 141.625 89.105) (width 0.25) (layer "F.Cu") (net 1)))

